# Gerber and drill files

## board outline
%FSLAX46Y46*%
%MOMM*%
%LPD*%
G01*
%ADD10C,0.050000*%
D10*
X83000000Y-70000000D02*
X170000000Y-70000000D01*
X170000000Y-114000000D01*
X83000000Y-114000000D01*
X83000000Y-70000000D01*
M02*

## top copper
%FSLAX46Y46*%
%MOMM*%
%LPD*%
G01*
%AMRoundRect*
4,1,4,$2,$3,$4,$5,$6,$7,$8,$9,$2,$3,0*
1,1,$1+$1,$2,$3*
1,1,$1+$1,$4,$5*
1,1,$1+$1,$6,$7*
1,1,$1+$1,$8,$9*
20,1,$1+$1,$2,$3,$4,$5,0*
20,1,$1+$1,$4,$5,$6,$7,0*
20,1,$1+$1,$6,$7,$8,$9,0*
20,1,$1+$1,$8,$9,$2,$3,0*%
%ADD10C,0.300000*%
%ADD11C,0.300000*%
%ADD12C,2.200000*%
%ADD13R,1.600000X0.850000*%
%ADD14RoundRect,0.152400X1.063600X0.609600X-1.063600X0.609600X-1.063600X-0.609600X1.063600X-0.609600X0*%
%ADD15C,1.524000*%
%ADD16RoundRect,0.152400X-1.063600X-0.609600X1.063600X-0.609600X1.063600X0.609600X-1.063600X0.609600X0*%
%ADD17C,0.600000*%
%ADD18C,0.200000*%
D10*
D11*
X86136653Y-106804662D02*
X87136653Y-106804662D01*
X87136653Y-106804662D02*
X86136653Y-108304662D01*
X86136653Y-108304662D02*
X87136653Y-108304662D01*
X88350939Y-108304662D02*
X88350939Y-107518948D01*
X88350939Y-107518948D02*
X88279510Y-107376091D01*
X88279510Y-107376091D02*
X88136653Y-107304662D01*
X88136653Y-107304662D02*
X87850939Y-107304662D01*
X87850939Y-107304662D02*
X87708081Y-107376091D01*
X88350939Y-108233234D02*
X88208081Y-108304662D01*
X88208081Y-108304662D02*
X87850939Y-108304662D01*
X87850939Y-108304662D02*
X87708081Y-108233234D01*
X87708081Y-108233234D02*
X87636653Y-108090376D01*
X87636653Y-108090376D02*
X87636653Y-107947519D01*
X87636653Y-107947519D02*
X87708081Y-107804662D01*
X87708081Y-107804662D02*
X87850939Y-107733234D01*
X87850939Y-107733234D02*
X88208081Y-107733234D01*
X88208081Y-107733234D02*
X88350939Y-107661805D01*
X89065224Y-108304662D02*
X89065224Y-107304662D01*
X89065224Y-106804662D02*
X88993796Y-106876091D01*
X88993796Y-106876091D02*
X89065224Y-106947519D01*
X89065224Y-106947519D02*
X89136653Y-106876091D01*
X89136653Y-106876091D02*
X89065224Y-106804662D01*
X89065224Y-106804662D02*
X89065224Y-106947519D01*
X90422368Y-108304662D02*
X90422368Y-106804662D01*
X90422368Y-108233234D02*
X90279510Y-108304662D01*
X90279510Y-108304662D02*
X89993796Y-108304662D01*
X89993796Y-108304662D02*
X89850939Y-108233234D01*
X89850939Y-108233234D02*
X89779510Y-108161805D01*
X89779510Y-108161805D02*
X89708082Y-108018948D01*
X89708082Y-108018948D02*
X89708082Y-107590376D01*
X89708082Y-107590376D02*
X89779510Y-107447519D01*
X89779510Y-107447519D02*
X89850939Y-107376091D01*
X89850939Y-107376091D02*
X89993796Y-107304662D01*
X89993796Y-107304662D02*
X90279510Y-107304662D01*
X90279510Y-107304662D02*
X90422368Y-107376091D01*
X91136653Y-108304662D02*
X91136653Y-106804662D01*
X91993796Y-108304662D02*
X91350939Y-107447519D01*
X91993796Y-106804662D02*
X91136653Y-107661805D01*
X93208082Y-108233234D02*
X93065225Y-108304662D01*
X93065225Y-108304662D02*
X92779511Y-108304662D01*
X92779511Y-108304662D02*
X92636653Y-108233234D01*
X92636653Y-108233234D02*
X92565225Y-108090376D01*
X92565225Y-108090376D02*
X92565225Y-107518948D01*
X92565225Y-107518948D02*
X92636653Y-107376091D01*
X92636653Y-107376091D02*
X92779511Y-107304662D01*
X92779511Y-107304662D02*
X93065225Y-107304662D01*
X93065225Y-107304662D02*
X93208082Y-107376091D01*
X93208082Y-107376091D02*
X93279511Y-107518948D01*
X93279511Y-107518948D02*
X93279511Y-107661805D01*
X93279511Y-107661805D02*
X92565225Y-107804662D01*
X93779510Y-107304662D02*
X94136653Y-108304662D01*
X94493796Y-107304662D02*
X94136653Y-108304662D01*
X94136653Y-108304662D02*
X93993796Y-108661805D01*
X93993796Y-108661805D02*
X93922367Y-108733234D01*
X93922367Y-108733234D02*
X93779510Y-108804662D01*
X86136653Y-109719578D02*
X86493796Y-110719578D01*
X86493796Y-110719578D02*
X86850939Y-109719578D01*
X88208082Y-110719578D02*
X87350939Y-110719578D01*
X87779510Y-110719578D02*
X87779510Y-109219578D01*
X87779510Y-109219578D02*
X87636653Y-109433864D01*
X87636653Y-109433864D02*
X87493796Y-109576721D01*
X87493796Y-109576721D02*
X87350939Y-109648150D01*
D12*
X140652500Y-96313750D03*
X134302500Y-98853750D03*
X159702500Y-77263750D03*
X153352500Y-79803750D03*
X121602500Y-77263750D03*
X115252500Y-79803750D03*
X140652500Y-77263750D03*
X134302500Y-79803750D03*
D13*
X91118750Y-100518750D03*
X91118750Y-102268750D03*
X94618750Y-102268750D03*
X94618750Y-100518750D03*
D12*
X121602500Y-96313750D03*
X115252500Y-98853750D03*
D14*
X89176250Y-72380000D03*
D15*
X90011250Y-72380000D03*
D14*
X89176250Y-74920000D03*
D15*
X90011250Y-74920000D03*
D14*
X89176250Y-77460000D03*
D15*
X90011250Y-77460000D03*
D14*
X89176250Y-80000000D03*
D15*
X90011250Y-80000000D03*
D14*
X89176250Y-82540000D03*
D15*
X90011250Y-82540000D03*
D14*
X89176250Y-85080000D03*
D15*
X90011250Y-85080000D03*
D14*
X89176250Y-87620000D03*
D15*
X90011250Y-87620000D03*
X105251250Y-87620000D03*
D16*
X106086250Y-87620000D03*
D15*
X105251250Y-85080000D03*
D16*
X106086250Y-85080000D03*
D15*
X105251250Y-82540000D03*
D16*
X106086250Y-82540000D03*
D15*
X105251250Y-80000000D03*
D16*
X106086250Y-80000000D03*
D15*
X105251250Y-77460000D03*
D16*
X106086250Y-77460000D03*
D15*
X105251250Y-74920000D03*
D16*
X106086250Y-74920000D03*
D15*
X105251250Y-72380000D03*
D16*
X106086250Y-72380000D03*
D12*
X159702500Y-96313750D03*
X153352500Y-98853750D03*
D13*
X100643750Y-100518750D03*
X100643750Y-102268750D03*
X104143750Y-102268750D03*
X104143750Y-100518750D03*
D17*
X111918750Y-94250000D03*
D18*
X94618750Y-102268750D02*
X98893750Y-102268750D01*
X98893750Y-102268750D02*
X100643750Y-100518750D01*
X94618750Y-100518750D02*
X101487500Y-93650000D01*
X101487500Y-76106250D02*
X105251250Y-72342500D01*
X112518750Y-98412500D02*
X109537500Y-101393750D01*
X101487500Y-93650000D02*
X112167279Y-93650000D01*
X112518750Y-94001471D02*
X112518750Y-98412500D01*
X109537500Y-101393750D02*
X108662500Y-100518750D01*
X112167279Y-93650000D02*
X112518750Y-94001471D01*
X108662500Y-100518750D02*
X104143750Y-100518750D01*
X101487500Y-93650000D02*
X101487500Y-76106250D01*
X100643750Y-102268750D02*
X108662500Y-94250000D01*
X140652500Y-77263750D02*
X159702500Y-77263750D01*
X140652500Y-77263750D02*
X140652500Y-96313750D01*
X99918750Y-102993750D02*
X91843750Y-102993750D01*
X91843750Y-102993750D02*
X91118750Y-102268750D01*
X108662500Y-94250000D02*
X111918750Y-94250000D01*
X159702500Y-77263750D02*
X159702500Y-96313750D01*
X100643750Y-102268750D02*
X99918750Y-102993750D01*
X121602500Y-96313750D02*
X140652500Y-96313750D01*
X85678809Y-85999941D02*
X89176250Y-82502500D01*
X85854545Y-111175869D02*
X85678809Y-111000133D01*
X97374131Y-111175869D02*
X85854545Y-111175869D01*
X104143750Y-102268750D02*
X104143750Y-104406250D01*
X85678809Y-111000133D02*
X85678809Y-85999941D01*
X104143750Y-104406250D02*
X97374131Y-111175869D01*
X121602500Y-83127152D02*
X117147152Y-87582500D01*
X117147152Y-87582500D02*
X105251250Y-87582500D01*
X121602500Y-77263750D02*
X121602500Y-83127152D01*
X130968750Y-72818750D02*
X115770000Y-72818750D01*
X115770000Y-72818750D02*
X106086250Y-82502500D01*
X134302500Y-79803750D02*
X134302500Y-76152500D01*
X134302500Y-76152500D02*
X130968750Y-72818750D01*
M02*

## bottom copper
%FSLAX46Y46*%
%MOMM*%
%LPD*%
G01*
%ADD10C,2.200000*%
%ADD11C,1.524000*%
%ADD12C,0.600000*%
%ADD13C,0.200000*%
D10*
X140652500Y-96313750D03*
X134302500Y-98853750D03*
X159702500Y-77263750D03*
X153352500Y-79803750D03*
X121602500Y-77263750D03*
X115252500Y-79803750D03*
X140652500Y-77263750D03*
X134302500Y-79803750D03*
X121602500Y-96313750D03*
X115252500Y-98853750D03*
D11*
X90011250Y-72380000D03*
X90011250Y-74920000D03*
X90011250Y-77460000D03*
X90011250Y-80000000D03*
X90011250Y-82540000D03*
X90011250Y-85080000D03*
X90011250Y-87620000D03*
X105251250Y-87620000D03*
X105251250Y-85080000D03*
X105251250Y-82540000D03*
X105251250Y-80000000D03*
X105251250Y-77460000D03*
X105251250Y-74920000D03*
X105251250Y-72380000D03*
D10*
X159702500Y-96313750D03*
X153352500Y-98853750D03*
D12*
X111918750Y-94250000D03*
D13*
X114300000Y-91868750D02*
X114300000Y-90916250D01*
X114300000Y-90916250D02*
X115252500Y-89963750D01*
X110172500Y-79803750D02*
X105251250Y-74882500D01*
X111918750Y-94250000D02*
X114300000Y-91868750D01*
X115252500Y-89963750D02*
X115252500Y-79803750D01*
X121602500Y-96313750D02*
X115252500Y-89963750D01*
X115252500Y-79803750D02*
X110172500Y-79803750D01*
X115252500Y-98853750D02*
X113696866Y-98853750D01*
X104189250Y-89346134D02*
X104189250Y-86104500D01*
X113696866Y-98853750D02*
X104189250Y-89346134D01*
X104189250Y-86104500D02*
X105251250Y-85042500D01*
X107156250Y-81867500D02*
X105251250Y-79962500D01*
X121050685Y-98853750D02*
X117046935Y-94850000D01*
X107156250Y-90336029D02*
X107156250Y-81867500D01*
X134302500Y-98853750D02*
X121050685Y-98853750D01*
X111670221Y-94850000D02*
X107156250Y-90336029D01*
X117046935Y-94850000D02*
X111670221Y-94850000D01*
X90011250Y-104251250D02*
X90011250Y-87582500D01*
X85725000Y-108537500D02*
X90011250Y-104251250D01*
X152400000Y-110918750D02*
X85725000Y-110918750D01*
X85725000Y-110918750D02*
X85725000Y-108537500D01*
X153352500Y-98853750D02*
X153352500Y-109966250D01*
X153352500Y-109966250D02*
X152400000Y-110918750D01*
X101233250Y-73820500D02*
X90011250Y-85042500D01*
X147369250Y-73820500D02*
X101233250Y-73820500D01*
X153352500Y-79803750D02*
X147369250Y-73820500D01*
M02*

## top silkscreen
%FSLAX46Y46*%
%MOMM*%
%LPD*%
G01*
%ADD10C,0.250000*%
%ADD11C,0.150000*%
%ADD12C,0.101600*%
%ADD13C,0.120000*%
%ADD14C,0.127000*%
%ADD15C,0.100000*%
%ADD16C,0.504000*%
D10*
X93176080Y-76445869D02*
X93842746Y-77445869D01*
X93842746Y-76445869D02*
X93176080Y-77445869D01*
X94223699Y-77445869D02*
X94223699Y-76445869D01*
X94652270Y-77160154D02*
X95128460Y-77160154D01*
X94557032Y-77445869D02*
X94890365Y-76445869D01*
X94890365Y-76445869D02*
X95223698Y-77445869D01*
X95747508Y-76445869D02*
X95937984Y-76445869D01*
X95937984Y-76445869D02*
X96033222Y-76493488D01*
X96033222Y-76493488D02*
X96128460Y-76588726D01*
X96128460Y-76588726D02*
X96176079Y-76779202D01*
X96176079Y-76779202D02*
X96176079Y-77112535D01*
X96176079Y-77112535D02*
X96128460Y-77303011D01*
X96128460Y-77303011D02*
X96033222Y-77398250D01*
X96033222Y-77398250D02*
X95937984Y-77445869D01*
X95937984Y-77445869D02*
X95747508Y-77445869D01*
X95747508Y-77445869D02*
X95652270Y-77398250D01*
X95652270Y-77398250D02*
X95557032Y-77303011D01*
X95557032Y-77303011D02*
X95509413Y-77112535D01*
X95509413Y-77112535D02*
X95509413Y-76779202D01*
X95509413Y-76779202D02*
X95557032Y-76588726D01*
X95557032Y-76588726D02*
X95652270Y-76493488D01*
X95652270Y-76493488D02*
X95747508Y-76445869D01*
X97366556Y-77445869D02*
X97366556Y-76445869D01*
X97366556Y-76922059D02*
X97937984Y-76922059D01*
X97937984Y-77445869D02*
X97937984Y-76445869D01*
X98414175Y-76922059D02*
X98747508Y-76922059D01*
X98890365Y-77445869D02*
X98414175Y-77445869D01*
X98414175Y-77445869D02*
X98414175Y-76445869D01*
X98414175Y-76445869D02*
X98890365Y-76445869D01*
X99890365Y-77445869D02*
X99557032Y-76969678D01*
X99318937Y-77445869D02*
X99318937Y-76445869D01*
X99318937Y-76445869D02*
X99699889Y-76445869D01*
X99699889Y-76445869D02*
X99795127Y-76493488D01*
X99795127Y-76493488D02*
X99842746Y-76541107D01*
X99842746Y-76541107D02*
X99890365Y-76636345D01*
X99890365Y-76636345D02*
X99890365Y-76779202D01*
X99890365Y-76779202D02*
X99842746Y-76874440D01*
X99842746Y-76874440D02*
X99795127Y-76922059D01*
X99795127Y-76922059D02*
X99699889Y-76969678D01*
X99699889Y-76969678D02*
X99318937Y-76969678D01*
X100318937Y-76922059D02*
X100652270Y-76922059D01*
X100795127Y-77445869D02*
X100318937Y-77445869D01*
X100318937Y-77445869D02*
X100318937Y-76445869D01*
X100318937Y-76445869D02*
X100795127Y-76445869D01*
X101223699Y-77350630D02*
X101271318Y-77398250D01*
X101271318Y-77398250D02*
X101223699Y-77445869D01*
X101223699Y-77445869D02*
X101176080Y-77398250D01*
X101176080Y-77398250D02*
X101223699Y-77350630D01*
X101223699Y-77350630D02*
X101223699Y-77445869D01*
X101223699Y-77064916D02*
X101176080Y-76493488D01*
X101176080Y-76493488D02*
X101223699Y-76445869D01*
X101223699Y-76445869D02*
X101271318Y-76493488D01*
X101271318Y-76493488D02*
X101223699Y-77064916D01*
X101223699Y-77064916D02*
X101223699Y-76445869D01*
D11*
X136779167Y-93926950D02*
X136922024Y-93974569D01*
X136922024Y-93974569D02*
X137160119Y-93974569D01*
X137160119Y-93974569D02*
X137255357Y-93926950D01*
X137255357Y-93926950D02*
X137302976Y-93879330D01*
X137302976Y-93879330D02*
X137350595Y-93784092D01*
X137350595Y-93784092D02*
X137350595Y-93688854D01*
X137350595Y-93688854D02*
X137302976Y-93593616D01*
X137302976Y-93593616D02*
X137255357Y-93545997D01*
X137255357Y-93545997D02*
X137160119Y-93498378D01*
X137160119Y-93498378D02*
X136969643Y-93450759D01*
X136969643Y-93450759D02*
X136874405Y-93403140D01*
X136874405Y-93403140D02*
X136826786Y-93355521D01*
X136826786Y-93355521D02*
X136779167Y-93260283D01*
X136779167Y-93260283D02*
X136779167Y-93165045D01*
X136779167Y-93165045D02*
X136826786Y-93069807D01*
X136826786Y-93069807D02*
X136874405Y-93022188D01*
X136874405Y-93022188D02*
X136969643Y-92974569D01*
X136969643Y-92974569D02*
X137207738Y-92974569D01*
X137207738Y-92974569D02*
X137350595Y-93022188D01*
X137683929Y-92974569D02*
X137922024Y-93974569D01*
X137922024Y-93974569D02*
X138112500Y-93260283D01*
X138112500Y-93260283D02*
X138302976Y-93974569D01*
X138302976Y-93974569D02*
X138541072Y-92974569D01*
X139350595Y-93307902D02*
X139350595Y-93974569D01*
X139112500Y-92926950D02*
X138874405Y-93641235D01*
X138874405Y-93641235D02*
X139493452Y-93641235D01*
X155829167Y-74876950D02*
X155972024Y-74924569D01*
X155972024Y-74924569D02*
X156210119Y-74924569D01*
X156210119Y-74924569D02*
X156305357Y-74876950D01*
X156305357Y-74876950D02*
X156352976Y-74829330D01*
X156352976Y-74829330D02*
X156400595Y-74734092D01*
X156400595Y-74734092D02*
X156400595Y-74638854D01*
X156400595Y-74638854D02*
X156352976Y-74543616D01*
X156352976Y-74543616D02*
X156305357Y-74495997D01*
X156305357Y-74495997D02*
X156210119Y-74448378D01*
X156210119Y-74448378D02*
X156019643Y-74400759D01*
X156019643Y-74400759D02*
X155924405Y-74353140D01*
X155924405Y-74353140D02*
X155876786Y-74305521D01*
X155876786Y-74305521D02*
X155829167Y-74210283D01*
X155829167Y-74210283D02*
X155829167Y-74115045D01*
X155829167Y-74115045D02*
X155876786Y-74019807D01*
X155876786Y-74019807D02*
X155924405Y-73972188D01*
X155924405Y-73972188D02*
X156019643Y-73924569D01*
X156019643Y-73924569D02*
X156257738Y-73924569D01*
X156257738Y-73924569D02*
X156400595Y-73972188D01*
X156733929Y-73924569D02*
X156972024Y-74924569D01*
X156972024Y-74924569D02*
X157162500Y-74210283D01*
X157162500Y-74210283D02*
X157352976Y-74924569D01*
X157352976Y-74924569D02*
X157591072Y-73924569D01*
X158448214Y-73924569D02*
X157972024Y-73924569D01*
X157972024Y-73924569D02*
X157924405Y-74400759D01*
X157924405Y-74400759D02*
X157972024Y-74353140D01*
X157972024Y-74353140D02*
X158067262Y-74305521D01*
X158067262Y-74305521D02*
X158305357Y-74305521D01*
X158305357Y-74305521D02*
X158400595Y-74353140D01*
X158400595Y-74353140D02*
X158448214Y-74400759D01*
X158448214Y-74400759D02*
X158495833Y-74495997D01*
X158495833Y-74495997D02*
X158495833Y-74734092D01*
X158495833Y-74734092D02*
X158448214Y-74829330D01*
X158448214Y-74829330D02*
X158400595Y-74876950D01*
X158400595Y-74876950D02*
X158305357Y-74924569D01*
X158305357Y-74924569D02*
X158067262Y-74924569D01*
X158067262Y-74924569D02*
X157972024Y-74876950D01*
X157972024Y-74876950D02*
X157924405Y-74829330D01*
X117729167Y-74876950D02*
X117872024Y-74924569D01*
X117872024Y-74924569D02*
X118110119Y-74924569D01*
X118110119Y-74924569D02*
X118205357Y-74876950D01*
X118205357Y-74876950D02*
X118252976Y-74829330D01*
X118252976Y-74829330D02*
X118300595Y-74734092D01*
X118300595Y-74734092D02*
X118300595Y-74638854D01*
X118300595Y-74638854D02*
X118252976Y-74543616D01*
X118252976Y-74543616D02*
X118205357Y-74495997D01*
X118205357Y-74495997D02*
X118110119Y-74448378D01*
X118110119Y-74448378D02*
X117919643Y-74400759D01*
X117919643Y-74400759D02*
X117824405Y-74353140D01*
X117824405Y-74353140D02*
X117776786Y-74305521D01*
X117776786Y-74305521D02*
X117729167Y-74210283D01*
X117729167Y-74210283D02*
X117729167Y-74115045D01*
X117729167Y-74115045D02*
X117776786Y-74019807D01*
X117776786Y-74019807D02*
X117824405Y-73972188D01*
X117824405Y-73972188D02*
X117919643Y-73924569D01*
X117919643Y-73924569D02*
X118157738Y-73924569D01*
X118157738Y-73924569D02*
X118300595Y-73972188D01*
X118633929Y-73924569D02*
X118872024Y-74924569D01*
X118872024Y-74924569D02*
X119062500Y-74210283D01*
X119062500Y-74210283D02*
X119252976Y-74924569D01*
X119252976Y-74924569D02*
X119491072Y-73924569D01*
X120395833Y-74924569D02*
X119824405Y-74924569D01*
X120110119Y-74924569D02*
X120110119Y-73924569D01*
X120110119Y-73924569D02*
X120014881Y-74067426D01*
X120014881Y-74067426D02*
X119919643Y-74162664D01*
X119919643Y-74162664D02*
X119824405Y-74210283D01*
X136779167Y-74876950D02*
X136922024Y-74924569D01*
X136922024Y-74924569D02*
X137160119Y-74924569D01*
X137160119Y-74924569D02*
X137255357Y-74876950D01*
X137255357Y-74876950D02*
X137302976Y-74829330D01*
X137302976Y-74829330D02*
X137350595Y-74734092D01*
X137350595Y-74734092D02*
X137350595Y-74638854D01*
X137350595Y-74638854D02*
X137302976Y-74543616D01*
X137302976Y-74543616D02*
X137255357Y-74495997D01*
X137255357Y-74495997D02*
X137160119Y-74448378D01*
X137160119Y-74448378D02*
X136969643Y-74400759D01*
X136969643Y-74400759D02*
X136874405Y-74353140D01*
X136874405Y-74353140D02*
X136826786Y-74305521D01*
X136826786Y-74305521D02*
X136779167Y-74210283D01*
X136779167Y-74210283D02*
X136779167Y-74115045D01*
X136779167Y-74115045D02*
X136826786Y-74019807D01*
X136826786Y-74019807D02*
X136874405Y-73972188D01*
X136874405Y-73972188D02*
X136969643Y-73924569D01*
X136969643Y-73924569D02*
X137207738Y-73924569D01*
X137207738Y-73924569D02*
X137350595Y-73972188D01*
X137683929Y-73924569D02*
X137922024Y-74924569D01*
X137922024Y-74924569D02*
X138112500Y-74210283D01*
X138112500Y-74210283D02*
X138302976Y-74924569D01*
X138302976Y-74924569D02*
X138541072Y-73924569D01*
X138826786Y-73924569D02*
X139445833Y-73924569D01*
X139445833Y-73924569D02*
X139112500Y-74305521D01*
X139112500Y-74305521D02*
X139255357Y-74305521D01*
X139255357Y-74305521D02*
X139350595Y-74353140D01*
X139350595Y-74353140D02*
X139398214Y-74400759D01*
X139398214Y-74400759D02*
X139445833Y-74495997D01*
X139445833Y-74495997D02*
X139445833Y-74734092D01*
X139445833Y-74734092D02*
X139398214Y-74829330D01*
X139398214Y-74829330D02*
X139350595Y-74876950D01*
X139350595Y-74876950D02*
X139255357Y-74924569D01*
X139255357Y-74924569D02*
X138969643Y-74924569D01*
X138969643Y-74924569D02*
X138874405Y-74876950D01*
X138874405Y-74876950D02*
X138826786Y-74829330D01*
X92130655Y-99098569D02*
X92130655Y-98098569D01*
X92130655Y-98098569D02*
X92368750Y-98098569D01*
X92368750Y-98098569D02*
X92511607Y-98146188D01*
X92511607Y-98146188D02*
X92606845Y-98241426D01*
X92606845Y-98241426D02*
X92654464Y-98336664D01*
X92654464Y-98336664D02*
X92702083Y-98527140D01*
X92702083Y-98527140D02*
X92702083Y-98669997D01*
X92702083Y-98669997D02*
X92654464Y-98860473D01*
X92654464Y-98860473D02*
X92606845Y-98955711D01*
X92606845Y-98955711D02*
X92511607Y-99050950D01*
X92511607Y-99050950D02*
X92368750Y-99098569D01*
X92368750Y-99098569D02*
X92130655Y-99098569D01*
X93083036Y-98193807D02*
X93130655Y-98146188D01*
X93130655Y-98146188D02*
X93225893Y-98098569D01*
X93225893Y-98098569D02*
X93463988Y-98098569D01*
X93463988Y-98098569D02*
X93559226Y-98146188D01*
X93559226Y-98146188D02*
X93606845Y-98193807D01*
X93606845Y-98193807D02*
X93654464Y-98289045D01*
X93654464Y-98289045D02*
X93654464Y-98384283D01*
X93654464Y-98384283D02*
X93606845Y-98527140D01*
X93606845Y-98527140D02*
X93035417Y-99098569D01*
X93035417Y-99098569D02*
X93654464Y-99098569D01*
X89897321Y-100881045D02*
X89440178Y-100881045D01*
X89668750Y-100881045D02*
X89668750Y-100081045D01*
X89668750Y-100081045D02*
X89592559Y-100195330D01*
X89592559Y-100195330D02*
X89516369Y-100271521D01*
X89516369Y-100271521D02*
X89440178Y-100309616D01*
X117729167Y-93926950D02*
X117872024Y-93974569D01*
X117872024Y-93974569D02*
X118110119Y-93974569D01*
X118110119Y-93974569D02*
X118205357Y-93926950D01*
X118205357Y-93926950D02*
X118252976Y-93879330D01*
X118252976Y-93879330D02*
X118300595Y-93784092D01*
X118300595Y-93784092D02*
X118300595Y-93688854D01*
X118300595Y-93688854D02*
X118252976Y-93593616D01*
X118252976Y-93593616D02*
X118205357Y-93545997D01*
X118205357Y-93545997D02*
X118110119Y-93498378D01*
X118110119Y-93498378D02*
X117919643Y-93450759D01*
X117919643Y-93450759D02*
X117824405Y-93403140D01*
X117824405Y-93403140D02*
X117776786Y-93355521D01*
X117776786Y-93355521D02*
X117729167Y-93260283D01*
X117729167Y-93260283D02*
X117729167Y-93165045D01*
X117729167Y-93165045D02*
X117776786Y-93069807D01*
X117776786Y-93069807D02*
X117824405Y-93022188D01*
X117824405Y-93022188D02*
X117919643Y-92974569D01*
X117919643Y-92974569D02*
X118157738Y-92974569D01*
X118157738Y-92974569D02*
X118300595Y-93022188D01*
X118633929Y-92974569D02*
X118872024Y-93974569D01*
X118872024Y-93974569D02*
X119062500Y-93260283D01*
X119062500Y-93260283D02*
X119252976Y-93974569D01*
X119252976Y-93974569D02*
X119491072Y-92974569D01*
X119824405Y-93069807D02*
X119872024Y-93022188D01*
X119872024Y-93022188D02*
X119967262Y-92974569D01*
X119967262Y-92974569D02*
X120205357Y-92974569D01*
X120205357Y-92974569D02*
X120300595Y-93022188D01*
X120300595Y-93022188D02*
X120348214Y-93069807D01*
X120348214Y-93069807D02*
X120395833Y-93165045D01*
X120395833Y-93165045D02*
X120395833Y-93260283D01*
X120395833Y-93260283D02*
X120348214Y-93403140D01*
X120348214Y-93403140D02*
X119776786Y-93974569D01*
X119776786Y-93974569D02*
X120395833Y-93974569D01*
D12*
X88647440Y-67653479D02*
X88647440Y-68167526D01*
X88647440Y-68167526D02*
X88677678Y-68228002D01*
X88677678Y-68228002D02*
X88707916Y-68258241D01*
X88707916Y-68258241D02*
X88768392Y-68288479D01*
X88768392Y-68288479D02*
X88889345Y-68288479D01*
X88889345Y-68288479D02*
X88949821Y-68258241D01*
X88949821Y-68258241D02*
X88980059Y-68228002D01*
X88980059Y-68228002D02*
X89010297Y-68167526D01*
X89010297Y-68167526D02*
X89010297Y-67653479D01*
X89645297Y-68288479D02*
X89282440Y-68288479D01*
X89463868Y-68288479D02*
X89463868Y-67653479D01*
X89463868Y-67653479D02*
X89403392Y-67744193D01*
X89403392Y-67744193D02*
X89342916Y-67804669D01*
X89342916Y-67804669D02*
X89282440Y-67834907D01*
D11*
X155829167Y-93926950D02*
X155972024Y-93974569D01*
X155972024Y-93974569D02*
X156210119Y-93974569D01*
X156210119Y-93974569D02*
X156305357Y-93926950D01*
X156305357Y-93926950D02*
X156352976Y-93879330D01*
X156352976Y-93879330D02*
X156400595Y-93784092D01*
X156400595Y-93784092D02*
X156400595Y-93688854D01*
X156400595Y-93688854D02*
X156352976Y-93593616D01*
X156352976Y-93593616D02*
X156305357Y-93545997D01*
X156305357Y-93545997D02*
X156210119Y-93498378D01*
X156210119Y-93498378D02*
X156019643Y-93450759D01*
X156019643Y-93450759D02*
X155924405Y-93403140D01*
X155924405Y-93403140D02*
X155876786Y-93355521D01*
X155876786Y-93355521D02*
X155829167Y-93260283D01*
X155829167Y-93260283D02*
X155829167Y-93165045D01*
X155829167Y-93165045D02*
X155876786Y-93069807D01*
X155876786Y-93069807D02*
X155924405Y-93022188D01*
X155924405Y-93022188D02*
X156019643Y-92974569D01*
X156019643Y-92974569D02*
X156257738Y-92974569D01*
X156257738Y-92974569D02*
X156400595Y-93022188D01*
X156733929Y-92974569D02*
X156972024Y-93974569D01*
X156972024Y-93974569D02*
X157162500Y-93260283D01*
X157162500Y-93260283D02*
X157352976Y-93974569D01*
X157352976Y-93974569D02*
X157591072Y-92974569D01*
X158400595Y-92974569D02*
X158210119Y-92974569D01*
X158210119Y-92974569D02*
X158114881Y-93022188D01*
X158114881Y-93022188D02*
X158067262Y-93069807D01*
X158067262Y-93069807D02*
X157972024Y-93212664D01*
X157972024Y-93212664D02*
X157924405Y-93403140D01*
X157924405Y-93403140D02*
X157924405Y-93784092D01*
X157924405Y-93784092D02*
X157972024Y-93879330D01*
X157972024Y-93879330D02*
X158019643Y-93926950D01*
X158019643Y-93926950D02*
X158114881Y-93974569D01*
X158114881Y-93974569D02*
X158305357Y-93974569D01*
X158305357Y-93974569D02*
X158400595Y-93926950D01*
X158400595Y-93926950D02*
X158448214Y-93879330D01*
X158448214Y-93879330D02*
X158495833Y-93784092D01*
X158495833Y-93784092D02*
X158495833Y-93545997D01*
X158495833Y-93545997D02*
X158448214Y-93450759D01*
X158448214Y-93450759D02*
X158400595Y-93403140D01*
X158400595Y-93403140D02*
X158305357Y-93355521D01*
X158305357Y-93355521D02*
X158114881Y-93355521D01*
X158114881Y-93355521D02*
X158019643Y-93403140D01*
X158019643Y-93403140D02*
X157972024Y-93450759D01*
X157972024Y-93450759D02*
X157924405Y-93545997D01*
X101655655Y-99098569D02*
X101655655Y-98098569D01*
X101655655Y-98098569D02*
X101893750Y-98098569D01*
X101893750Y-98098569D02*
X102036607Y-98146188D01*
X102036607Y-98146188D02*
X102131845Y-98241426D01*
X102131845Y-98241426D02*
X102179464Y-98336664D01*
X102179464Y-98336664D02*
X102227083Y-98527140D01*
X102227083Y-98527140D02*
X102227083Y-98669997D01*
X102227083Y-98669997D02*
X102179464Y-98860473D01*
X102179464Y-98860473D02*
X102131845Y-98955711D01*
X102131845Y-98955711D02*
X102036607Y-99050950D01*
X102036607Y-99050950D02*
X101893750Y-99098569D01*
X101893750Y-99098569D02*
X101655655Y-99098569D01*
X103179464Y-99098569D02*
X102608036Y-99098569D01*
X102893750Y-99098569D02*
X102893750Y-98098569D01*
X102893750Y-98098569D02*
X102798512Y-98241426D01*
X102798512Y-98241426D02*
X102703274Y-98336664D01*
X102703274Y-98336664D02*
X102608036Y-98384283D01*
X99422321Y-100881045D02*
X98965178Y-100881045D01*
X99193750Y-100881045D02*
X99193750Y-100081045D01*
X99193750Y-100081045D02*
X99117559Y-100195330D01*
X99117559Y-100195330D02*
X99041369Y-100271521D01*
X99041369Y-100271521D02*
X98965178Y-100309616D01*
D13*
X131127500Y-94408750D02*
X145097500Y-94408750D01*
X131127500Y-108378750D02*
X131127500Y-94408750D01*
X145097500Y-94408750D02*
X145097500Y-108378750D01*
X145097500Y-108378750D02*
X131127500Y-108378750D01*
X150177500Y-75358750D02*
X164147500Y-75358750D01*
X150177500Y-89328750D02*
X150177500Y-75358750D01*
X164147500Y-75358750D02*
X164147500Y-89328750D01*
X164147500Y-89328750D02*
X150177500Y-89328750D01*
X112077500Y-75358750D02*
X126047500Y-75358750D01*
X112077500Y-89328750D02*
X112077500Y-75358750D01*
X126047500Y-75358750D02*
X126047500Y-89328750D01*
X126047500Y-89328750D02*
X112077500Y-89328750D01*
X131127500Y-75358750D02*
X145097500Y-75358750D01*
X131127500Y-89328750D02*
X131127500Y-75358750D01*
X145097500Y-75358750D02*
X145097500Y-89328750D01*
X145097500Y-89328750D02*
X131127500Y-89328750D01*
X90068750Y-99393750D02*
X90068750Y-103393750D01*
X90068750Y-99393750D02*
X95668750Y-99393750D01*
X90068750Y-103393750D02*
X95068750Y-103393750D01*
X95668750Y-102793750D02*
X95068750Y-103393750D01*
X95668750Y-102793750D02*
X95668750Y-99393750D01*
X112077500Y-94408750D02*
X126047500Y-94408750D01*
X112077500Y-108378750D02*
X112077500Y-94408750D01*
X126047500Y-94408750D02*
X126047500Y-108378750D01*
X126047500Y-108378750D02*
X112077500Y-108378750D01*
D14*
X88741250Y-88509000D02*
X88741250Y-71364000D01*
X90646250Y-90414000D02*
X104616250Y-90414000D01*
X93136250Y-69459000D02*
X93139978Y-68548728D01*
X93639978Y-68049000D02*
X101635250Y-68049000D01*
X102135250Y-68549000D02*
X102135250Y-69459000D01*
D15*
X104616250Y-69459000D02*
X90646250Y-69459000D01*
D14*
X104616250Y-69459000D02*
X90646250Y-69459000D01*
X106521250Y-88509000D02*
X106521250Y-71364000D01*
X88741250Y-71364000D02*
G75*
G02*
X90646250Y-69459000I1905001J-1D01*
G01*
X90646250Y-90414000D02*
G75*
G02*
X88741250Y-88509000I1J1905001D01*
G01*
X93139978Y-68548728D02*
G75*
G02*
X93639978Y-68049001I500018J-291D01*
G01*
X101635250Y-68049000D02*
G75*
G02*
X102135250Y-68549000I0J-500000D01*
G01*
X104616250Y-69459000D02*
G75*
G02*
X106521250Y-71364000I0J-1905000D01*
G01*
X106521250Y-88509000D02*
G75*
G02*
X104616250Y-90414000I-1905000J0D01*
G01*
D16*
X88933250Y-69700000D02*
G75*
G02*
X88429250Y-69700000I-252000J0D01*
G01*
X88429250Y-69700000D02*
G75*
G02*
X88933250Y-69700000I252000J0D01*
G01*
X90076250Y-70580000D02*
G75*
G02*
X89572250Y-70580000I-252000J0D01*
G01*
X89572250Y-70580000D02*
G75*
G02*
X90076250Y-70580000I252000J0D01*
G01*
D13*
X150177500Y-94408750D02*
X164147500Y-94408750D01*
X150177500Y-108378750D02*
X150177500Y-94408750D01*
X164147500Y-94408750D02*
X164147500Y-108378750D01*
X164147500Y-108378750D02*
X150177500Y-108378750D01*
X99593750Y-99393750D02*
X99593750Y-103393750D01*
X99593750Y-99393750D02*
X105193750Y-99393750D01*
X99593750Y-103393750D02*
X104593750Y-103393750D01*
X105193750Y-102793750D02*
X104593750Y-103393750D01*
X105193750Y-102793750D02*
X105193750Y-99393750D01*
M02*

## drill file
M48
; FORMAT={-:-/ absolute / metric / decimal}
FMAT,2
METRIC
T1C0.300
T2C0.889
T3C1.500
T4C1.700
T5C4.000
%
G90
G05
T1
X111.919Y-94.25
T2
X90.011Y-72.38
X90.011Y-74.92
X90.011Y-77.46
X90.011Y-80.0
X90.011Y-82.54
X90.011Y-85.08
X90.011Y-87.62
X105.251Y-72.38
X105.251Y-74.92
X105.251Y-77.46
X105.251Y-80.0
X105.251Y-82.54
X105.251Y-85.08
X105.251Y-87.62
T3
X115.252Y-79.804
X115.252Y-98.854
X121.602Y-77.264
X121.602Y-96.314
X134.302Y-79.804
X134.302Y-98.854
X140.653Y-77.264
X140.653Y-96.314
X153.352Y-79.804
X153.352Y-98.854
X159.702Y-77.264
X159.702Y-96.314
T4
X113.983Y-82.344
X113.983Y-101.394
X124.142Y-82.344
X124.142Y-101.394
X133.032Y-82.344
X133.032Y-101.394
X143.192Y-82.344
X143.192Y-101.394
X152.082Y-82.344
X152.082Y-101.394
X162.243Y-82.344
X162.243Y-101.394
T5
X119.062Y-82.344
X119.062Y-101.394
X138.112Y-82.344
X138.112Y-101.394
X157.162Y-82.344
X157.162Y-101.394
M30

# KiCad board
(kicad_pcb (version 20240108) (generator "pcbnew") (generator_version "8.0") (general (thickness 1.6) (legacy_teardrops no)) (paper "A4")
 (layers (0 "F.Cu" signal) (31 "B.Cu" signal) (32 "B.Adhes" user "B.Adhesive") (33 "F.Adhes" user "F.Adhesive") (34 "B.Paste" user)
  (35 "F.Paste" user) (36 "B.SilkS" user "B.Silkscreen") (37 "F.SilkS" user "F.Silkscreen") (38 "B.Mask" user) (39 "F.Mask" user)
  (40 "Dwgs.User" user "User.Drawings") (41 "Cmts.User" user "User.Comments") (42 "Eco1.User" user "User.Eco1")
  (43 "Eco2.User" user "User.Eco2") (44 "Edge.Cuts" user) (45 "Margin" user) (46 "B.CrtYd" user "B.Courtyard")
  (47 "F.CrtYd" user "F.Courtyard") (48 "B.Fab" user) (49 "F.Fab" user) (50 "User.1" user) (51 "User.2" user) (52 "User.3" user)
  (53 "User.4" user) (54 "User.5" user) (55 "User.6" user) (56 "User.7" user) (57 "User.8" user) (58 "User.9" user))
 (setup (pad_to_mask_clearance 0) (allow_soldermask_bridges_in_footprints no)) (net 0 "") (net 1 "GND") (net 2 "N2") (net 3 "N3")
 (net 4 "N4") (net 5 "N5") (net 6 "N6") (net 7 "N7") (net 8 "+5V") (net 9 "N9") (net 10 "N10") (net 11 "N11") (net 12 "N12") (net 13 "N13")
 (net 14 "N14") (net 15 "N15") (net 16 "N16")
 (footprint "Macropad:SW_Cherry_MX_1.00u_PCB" (layer "F.Cu") (at 140.6525 96.31375)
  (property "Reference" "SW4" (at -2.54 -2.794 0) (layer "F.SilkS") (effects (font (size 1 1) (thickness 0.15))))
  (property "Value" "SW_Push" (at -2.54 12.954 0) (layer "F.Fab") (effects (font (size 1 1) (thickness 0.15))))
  (fp_line (start -9.525 -1.905) (end 4.445 -1.905) (stroke (width 0.12) (type solid)) (layer "F.SilkS"))
  (fp_line (start -9.525 12.065) (end -9.525 -1.905) (stroke (width 0.12) (type solid)) (layer "F.SilkS"))
  (fp_line (start 4.445 -1.905) (end 4.445 12.065) (stroke (width 0.12) (type solid)) (layer "F.SilkS"))
  (fp_line (start 4.445 12.065) (end -9.525 12.065) (stroke (width 0.12) (type solid)) (layer "F.SilkS"))
  (pad "" np_thru_hole circle (at -7.62 5.08) (size 1.7 1.7) (drill 1.7) (layers "*.Cu" "*.Mask"))
  (pad "" np_thru_hole circle (at -2.54 5.08) (size 4 4) (drill 4) (layers "*.Cu" "*.Mask"))
  (pad "" np_thru_hole circle (at 2.54 5.08) (size 1.7 1.7) (drill 1.7) (layers "*.Cu" "*.Mask"))
  (pad "1" thru_hole circle (at 0 0) (size 2.2 2.2) (drill 1.5) (layers "*.Cu" "*.Mask") (remove_unused_layers no) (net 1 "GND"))
  (pad "2" thru_hole circle (at -6.35 2.54) (size 2.2 2.2) (drill 1.5) (layers "*.Cu" "*.Mask") (remove_unused_layers no) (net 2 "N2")))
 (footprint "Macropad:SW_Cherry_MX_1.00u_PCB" (layer "F.Cu") (at 159.7025 77.26375)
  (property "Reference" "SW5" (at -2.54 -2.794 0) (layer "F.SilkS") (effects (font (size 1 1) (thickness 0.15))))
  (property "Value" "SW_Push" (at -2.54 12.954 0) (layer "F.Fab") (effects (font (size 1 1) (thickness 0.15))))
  (fp_line (start -9.525 -1.905) (end 4.445 -1.905) (stroke (width 0.12) (type solid)) (layer "F.SilkS"))
  (fp_line (start -9.525 12.065) (end -9.525 -1.905) (stroke (width 0.12) (type solid)) (layer "F.SilkS"))
  (fp_line (start 4.445 -1.905) (end 4.445 12.065) (stroke (width 0.12) (type solid)) (layer "F.SilkS"))
  (fp_line (start 4.445 12.065) (end -9.525 12.065) (stroke (width 0.12) (type solid)) (layer "F.SilkS"))
  (pad "" np_thru_hole circle (at -7.62 5.08) (size 1.7 1.7) (drill 1.7) (layers "*.Cu" "*.Mask"))
  (pad "" np_thru_hole circle (at -2.54 5.08) (size 4 4) (drill 4) (layers "*.Cu" "*.Mask"))
  (pad "" np_thru_hole circle (at 2.54 5.08) (size 1.7 1.7) (drill 1.7) (layers "*.Cu" "*.Mask"))
  (pad "1" thru_hole circle (at 0 0) (size 2.2 2.2) (drill 1.5) (layers "*.Cu" "*.Mask") (remove_unused_layers no) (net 1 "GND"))
  (pad "2" thru_hole circle (at -6.35 2.54) (size 2.2 2.2) (drill 1.5) (layers "*.Cu" "*.Mask") (remove_unused_layers no) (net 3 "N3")))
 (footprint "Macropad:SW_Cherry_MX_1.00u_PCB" (layer "F.Cu") (at 121.6025 77.26375)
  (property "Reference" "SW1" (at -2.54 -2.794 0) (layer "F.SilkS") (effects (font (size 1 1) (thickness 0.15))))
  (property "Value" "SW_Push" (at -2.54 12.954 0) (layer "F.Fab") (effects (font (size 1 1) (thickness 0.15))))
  (fp_line (start -9.525 -1.905) (end 4.445 -1.905) (stroke (width 0.12) (type solid)) (layer "F.SilkS"))
  (fp_line (start -9.525 12.065) (end -9.525 -1.905) (stroke (width 0.12) (type solid)) (layer "F.SilkS"))
  (fp_line (start 4.445 -1.905) (end 4.445 12.065) (stroke (width 0.12) (type solid)) (layer "F.SilkS"))
  (fp_line (start 4.445 12.065) (end -9.525 12.065) (stroke (width 0.12) (type solid)) (layer "F.SilkS"))
  (pad "" np_thru_hole circle (at -7.62 5.08) (size 1.7 1.7) (drill 1.7) (layers "*.Cu" "*.Mask"))
  (pad "" np_thru_hole circle (at -2.54 5.08) (size 4 4) (drill 4) (layers "*.Cu" "*.Mask"))
  (pad "" np_thru_hole circle (at 2.54 5.08) (size 1.7 1.7) (drill 1.7) (layers "*.Cu" "*.Mask"))
  (pad "1" thru_hole circle (at 0 0) (size 2.2 2.2) (drill 1.5) (layers "*.Cu" "*.Mask") (remove_unused_layers no) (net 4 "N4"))
  (pad "2" thru_hole circle (at -6.35 2.54) (size 2.2 2.2) (drill 1.5) (layers "*.Cu" "*.Mask") (remove_unused_layers no) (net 1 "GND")))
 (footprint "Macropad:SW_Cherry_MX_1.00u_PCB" (layer "F.Cu") (at 140.6525 77.26375)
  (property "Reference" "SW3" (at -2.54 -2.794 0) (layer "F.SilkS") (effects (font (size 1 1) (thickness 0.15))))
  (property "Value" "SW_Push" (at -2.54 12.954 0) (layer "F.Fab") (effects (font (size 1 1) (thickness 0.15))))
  (fp_line (start -9.525 -1.905) (end 4.445 -1.905) (stroke (width 0.12) (type solid)) (layer "F.SilkS"))
  (fp_line (start -9.525 12.065) (end -9.525 -1.905) (stroke (width 0.12) (type solid)) (layer "F.SilkS"))
  (fp_line (start 4.445 -1.905) (end 4.445 12.065) (stroke (width 0.12) (type solid)) (layer "F.SilkS"))
  (fp_line (start 4.445 12.065) (end -9.525 12.065) (stroke (width 0.12) (type solid)) (layer "F.SilkS"))
  (pad "" np_thru_hole circle (at -7.62 5.08) (size 1.7 1.7) (drill 1.7) (layers "*.Cu" "*.Mask"))
  (pad "" np_thru_hole circle (at -2.54 5.08) (size 4 4) (drill 4) (layers "*.Cu" "*.Mask"))
  (pad "" np_thru_hole circle (at 2.54 5.08) (size 1.7 1.7) (drill 1.7) (layers "*.Cu" "*.Mask"))
  (pad "1" thru_hole circle (at 0 0) (size 2.2 2.2) (drill 1.5) (layers "*.Cu" "*.Mask") (remove_unused_layers no) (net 1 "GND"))
  (pad "2" thru_hole circle (at -6.35 2.54) (size 2.2 2.2) (drill 1.5) (layers "*.Cu" "*.Mask") (remove_unused_layers no) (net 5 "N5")))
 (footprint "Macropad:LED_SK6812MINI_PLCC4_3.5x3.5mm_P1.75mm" (layer "F.Cu") (at 92.86875 101.39375)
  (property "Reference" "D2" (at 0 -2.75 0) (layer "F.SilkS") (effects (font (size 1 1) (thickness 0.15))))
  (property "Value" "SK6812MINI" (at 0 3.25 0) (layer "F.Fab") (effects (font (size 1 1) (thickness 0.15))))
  (fp_line (start -2.8 -2) (end -2.8 2) (stroke (width 0.12) (type default)) (layer "F.SilkS"))
  (fp_line (start -2.8 -2) (end 2.8 -2) (stroke (width 0.12) (type solid)) (layer "F.SilkS"))
  (fp_line (start -2.8 2) (end 2.2 2) (stroke (width 0.12) (type solid)) (layer "F.SilkS"))
  (fp_line (start 2.8 1.4) (end 2.2 2) (stroke (width 0.12) (type default)) (layer "F.SilkS"))
  (fp_line (start 2.8 1.4) (end 2.8 -2) (stroke (width 0.12) (type solid)) (layer "F.SilkS"))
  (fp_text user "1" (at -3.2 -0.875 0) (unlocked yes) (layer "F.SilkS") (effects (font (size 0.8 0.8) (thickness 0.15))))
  (pad "1" smd rect (at -1.75 -0.875) (size 1.6 0.85) (layers "F.Cu" "F.Paste" "F.Mask") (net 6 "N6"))
  (pad "2" smd rect (at -1.75 0.875) (size 1.6 0.85) (layers "F.Cu" "F.Paste" "F.Mask") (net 1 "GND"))
  (pad "3" smd rect (at 1.75 0.875) (size 1.6 0.85) (layers "F.Cu" "F.Paste" "F.Mask") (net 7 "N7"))
  (pad "4" smd rect (at 1.75 -0.875) (size 1.6 0.85) (layers "F.Cu" "F.Paste" "F.Mask") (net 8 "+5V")))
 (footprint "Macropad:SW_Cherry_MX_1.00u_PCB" (layer "F.Cu") (at 121.6025 96.31375)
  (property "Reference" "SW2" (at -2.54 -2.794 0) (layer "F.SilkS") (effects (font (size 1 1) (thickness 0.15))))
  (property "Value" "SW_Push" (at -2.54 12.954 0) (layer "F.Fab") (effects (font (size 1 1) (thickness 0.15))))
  (fp_line (start -9.525 -1.905) (end 4.445 -1.905) (stroke (width 0.12) (type solid)) (layer "F.SilkS"))
  (fp_line (start -9.525 12.065) (end -9.525 -1.905) (stroke (width 0.12) (type solid)) (layer "F.SilkS"))
  (fp_line (start 4.445 -1.905) (end 4.445 12.065) (stroke (width 0.12) (type solid)) (layer "F.SilkS"))
  (fp_line (start 4.445 12.065) (end -9.525 12.065) (stroke (width 0.12) (type solid)) (layer "F.SilkS"))
  (pad "" np_thru_hole circle (at -7.62 5.08) (size 1.7 1.7) (drill 1.7) (layers "*.Cu" "*.Mask"))
  (pad "" np_thru_hole circle (at -2.54 5.08) (size 4 4) (drill 4) (layers "*.Cu" "*.Mask"))
  (pad "" np_thru_hole circle (at 2.54 5.08) (size 1.7 1.7) (drill 1.7) (layers "*.Cu" "*.Mask"))
  (pad "1" thru_hole circle (at 0 0) (size 2.2 2.2) (drill 1.5) (layers "*.Cu" "*.Mask") (remove_unused_layers no) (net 1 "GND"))
  (pad "2" thru_hole circle (at -6.35 2.54) (size 2.2 2.2) (drill 1.5) (layers "*.Cu" "*.Mask") (remove_unused_layers no) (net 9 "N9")))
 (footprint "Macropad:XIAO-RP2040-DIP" (layer "F.Cu") (at 97.63125 80)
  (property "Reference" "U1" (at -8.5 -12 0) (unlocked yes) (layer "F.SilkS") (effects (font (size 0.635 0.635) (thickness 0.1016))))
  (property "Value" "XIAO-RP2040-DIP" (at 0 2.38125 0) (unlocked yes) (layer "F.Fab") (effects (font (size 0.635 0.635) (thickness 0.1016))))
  (fp_line (start -8.89 8.509) (end -8.89 -8.636) (stroke (width 0.127) (type solid)) (layer "F.SilkS"))
  (fp_line (start -6.985 10.414) (end 6.985 10.414) (stroke (width 0.127) (type solid)) (layer "F.SilkS"))
  (fp_line (start -4.495 -10.541) (end -4.491272 -11.451272) (stroke (width 0.127) (type solid)) (layer "F.SilkS"))
  (fp_line (start -3.991272 -11.951) (end 4.004 -11.951) (stroke (width 0.127) (type solid)) (layer "F.SilkS"))
  (fp_line (start 4.504 -11.451) (end 4.504 -10.541) (stroke (width 0.127) (type solid)) (layer "F.SilkS"))
  (fp_line (start 6.985 -10.541) (end -6.985 -10.541) (stroke (width 0.1) (type solid)) (layer "F.SilkS"))
  (fp_line (start 6.985 -10.541) (end -6.985 -10.541) (stroke (width 0.127) (type solid)) (layer "F.SilkS"))
  (fp_line (start 8.89 8.509) (end 8.89 -8.636) (stroke (width 0.127) (type solid)) (layer "F.SilkS"))
  (fp_arc (start -8.89 -8.636) (mid -8.332038 -9.983038) (end -6.985 -10.541) (stroke (width 0.127) (type solid)) (layer "F.SilkS"))
  (fp_arc (start -6.985 10.414) (mid -8.332038 9.856038) (end -8.89 8.509) (stroke (width 0.127) (type solid)) (layer "F.SilkS"))
  (fp_arc (start -4.491272 -11.451272) (mid -4.344724 -11.804644) (end -3.991272 -11.951) (stroke (width 0.127) (type default))
   (layer "F.SilkS"))
  (fp_arc (start 4.004 -11.951) (mid 4.357553 -11.804553) (end 4.504 -11.451) (stroke (width 0.127) (type default)) (layer "F.SilkS"))
  (fp_arc (start 6.985 -10.541) (mid 8.332038 -9.983038) (end 8.89 -8.636) (stroke (width 0.127) (type solid)) (layer "F.SilkS"))
  (fp_arc (start 8.89 8.509) (mid 8.332038 9.856038) (end 6.985 10.414) (stroke (width 0.127) (type solid)) (layer "F.SilkS"))
  (fp_circle (center -8.95 -10.3) (end -8.95 -10.554) (stroke (width 0.5) (type solid)) (fill solid) (layer "F.SilkS"))
  (fp_circle (center -7.807 -9.42) (end -7.807 -9.674) (stroke (width 0.5) (type solid)) (fill solid) (layer "F.SilkS"))
  (pad "1" smd roundrect (at -8.455 -7.62 180) (size 2.432 1.524) (layers "F.Cu" "F.Mask") (roundrect_rratio 0.1) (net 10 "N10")
   (thermal_bridge_angle 45))
  (pad "1" thru_hole circle (at -7.62 -7.62 180) (size 1.524 1.524) (drill 0.889) (layers "*.Cu" "*.Mask") (remove_unused_layers no)
   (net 10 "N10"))
  (pad "2" smd roundrect (at -8.455 -5.08 180) (size 2.432 1.524) (layers "F.Cu" "F.Mask") (roundrect_rratio 0.1) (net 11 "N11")
   (thermal_bridge_angle 45))
  (pad "2" thru_hole circle (at -7.62 -5.08 180) (size 1.524 1.524) (drill 0.889) (layers "*.Cu" "*.Mask") (remove_unused_layers no)
   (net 11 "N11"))
  (pad "3" smd roundrect (at -8.455 -2.54 180) (size 2.432 1.524) (layers "F.Cu" "F.Mask") (roundrect_rratio 0.1) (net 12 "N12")
   (thermal_bridge_angle 45))
  (pad "3" thru_hole circle (at -7.62 -2.54 180) (size 1.524 1.524) (drill 0.889) (layers "*.Cu" "*.Mask") (remove_unused_layers no)
   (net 12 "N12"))
  (pad "4" smd roundrect (at -8.455 0 180) (size 2.432 1.524) (layers "F.Cu" "F.Mask") (roundrect_rratio 0.1) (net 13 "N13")
   (thermal_bridge_angle 45))
  (pad "4" thru_hole circle (at -7.62 0 180) (size 1.524 1.524) (drill 0.889) (layers "*.Cu" "*.Mask") (remove_unused_layers no)
   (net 13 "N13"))
  (pad "5" smd roundrect (at -8.455 2.54 180) (size 2.432 1.524) (layers "F.Cu" "F.Mask") (roundrect_rratio 0.1) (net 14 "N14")
   (thermal_bridge_angle 45))
  (pad "5" thru_hole circle (at -7.62 2.54 180) (size 1.524 1.524) (drill 0.889) (layers "*.Cu" "*.Mask") (remove_unused_layers no)
   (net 14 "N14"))
  (pad "6" smd roundrect (at -8.455 5.08 180) (size 2.432 1.524) (layers "F.Cu" "F.Mask") (roundrect_rratio 0.1) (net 3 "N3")
   (thermal_bridge_angle 45))
  (pad "6" thru_hole circle (at -7.62 5.08 180) (size 1.524 1.524) (drill 0.889) (layers "*.Cu" "*.Mask") (remove_unused_layers no)
   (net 3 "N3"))
  (pad "7" smd roundrect (at -8.455 7.62 180) (size 2.432 1.524) (layers "F.Cu" "F.Mask") (roundrect_rratio 0.1) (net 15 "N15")
   (thermal_bridge_angle 45))
  (pad "7" thru_hole circle (at -7.62 7.62 180) (size 1.524 1.524) (drill 0.889) (layers "*.Cu" "*.Mask") (remove_unused_layers no)
   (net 15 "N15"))
  (pad "8" thru_hole circle (at 7.62 7.62) (size 1.524 1.524) (drill 0.889) (layers "*.Cu" "*.Mask") (remove_unused_layers no) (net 4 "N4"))
  (pad "8" smd roundrect (at 8.455 7.62) (size 2.432 1.524) (layers "F.Cu" "F.Mask") (roundrect_rratio 0.1) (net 4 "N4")
   (thermal_bridge_angle 45))
  (pad "9" thru_hole circle (at 7.62 5.08) (size 1.524 1.524) (drill 0.889) (layers "*.Cu" "*.Mask") (remove_unused_layers no) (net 9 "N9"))
  (pad "9" smd roundrect (at 8.455 5.08) (size 2.432 1.524) (layers "F.Cu" "F.Mask") (roundrect_rratio 0.1) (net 9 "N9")
   (thermal_bridge_angle 45))
  (pad "10" thru_hole circle (at 7.62 2.54) (size 1.524 1.524) (drill 0.889) (layers "*.Cu" "*.Mask") (remove_unused_layers no) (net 5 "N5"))
  (pad "10" smd roundrect (at 8.455 2.54) (size 2.432 1.524) (layers "F.Cu" "F.Mask") (roundrect_rratio 0.1) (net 5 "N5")
   (thermal_bridge_angle 45))
  (pad "11" thru_hole circle (at 7.62 0) (size 1.524 1.524) (drill 0.889) (layers "*.Cu" "*.Mask") (remove_unused_layers no) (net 2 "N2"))
  (pad "11" smd roundrect (at 8.455 0) (size 2.432 1.524) (layers "F.Cu" "F.Mask") (roundrect_rratio 0.1) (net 2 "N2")
   (thermal_bridge_angle 45))
  (pad "12" thru_hole circle (at 7.62 -2.54) (size 1.524 1.524) (drill 0.889) (layers "*.Cu" "*.Mask") (remove_unused_layers no)
   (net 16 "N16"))
  (pad "12" smd roundrect (at 8.455 -2.54) (size 2.432 1.524) (layers "F.Cu" "F.Mask") (roundrect_rratio 0.1) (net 16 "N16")
   (thermal_bridge_angle 45))
  (pad "13" thru_hole circle (at 7.62 -5.08) (size 1.524 1.524) (drill 0.889) (layers "*.Cu" "*.Mask") (remove_unused_layers no)
   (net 1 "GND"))
  (pad "13" smd roundrect (at 8.455 -5.08) (size 2.432 1.524) (layers "F.Cu" "F.Mask") (roundrect_rratio 0.1) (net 1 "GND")
   (thermal_bridge_angle 45))
  (pad "14" thru_hole circle (at 7.62 -7.62) (size 1.524 1.524) (drill 0.889) (layers "*.Cu" "*.Mask") (remove_unused_layers no)
   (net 8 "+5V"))
  (pad "14" smd roundrect (at 8.455 -7.62) (size 2.432 1.524) (layers "F.Cu" "F.Mask") (roundrect_rratio 0.1) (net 8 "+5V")
   (thermal_bridge_angle 45)))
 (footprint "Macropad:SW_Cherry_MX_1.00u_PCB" (layer "F.Cu") (at 159.7025 96.31375)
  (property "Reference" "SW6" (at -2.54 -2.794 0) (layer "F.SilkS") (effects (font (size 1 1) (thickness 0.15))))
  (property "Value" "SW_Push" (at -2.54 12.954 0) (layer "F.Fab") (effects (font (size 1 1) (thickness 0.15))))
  (fp_line (start -9.525 -1.905) (end 4.445 -1.905) (stroke (width 0.12) (type solid)) (layer "F.SilkS"))
  (fp_line (start -9.525 12.065) (end -9.525 -1.905) (stroke (width 0.12) (type solid)) (layer "F.SilkS"))
  (fp_line (start 4.445 -1.905) (end 4.445 12.065) (stroke (width 0.12) (type solid)) (layer "F.SilkS"))
  (fp_line (start 4.445 12.065) (end -9.525 12.065) (stroke (width 0.12) (type solid)) (layer "F.SilkS"))
  (pad "" np_thru_hole circle (at -7.62 5.08) (size 1.7 1.7) (drill 1.7) (layers "*.Cu" "*.Mask"))
  (pad "" np_thru_hole circle (at -2.54 5.08) (size 4 4) (drill 4) (layers "*.Cu" "*.Mask"))
  (pad "" np_thru_hole circle (at 2.54 5.08) (size 1.7 1.7) (drill 1.7) (layers "*.Cu" "*.Mask"))
  (pad "1" thru_hole circle (at 0 0) (size 2.2 2.2) (drill 1.5) (layers "*.Cu" "*.Mask") (remove_unused_layers no) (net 1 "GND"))
  (pad "2" thru_hole circle (at -6.35 2.54) (size 2.2 2.2) (drill 1.5) (layers "*.Cu" "*.Mask") (remove_unused_layers no) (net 15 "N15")))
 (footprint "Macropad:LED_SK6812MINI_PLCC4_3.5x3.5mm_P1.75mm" (layer "F.Cu") (at 102.39375 101.39375)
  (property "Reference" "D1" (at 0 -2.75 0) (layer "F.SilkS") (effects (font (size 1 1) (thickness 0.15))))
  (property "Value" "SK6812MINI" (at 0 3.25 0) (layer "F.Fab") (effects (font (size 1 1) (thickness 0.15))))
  (fp_line (start -2.8 -2) (end -2.8 2) (stroke (width 0.12) (type default)) (layer "F.SilkS"))
  (fp_line (start -2.8 -2) (end 2.8 -2) (stroke (width 0.12) (type solid)) (layer "F.SilkS"))
  (fp_line (start -2.8 2) (end 2.2 2) (stroke (width 0.12) (type solid)) (layer "F.SilkS"))
  (fp_line (start 2.8 1.4) (end 2.2 2) (stroke (width 0.12) (type default)) (layer "F.SilkS"))
  (fp_line (start 2.8 1.4) (end 2.8 -2) (stroke (width 0.12) (type solid)) (layer "F.SilkS"))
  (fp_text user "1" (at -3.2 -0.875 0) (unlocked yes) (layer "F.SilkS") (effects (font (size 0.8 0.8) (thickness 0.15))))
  (pad "1" smd rect (at -1.75 -0.875) (size 1.6 0.85) (layers "F.Cu" "F.Paste" "F.Mask") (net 7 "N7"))
  (pad "2" smd rect (at -1.75 0.875) (size 1.6 0.85) (layers "F.Cu" "F.Paste" "F.Mask") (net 1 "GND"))
  (pad "3" smd rect (at 1.75 0.875) (size 1.6 0.85) (layers "F.Cu" "F.Paste" "F.Mask") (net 14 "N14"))
  (pad "4" smd rect (at 1.75 -0.875) (size 1.6 0.85) (layers "F.Cu" "F.Paste" "F.Mask") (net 8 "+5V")))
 (gr_rect (start 83 70) (end 170 114) (stroke (width 0.05) (type default)) (fill none) (layer "Edge.Cuts"))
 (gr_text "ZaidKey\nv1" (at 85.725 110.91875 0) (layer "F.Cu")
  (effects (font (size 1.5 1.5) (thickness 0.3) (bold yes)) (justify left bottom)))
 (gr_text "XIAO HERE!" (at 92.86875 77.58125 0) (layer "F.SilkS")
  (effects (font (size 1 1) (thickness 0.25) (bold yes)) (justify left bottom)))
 (segment (start 94.61875 102.26875) (end 98.89375 102.26875) (width 0.2) (layer "F.Cu") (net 7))
 (segment (start 98.89375 102.26875) (end 100.64375 100.51875) (width 0.2) (layer "F.Cu") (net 7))
 (segment (start 94.61875 100.51875) (end 101.4875 93.65) (width 0.2) (layer "F.Cu") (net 8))
 (segment (start 101.4875 76.10625) (end 105.25125 72.3425) (width 0.2) (layer "F.Cu") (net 8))
 (segment (start 112.51875 98.4125) (end 109.5375 101.39375) (width 0.2) (layer "F.Cu") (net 8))
 (segment (start 101.4875 93.65) (end 112.167279 93.65) (width 0.2) (layer "F.Cu") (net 8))
 (segment (start 112.51875 94.001471) (end 112.51875 98.4125) (width 0.2) (layer "F.Cu") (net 8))
 (segment (start 109.5375 101.39375) (end 108.6625 100.51875) (width 0.2) (layer "F.Cu") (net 8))
 (segment (start 112.167279 93.65) (end 112.51875 94.001471) (width 0.2) (layer "F.Cu") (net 8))
 (segment (start 108.6625 100.51875) (end 104.14375 100.51875) (width 0.2) (layer "F.Cu") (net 8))
 (segment (start 101.4875 93.65) (end 101.4875 76.10625) (width 0.2) (layer "F.Cu") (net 8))
 (segment (start 100.64375 102.26875) (end 108.6625 94.25) (width 0.2) (layer "F.Cu") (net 1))
 (segment (start 140.6525 77.26375) (end 159.7025 77.26375) (width 0.2) (layer "F.Cu") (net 1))
 (segment (start 140.6525 77.26375) (end 140.6525 96.31375) (width 0.2) (layer "F.Cu") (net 1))
 (segment (start 99.91875 102.99375) (end 91.84375 102.99375) (width 0.2) (layer "F.Cu") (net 1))
 (segment (start 91.84375 102.99375) (end 91.11875 102.26875) (width 0.2) (layer "F.Cu") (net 1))
 (segment (start 108.6625 94.25) (end 111.91875 94.25) (width 0.2) (layer "F.Cu") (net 1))
 (segment (start 159.7025 77.26375) (end 159.7025 96.31375) (width 0.2) (layer "F.Cu") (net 1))
 (segment (start 100.64375 102.26875) (end 99.91875 102.99375) (width 0.2) (layer "F.Cu") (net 1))
 (segment (start 121.6025 96.31375) (end 140.6525 96.31375) (width 0.2) (layer "F.Cu") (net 1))
 (via (at 111.91875 94.25) (size 0.6) (drill 0.3) (layers "F.Cu" "B.Cu") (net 1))
 (segment (start 114.3 91.86875) (end 114.3 90.91625) (width 0.2) (layer "B.Cu") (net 1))
 (segment (start 114.3 90.91625) (end 115.2525 89.96375) (width 0.2) (layer "B.Cu") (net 1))
 (segment (start 110.1725 79.80375) (end 105.25125 74.8825) (width 0.2) (layer "B.Cu") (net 1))
 (segment (start 111.91875 94.25) (end 114.3 91.86875) (width 0.2) (layer "B.Cu") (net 1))
 (segment (start 115.2525 89.96375) (end 115.2525 79.80375) (width 0.2) (layer "B.Cu") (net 1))
 (segment (start 121.6025 96.31375) (end 115.2525 89.96375) (width 0.2) (layer "B.Cu") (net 1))
 (segment (start 115.2525 79.80375) (end 110.1725 79.80375) (width 0.2) (layer "B.Cu") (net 1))
 (segment (start 85.678809 85.999941) (end 89.17625 82.5025) (width 0.2) (layer "F.Cu") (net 14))
 (segment (start 85.854545 111.175869) (end 85.678809 111.000133) (width 0.2) (layer "F.Cu") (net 14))
 (segment (start 97.374131 111.175869) (end 85.854545 111.175869) (width 0.2) (layer "F.Cu") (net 14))
 (segment (start 104.14375 102.26875) (end 104.14375 104.40625) (width 0.2) (layer "F.Cu") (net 14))
 (segment (start 85.678809 111.000133) (end 85.678809 85.999941) (width 0.2) (layer "F.Cu") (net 14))
 (segment (start 104.14375 104.40625) (end 97.374131 111.175869) (width 0.2) (layer "F.Cu") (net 14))
 (segment (start 121.6025 83.127152) (end 117.147152 87.5825) (width 0.2) (layer "F.Cu") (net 4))
 (segment (start 117.147152 87.5825) (end 105.25125 87.5825) (width 0.2) (layer "F.Cu") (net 4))
 (segment (start 121.6025 77.26375) (end 121.6025 83.127152) (width 0.2) (layer "F.Cu") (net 4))
 (segment (start 115.2525 98.85375) (end 113.696866 98.85375) (width 0.2) (layer "B.Cu") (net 9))
 (segment (start 104.18925 89.346134) (end 104.18925 86.1045) (width 0.2) (layer "B.Cu") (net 9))
 (segment (start 113.696866 98.85375) (end 104.18925 89.346134) (width 0.2) (layer "B.Cu") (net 9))
 (segment (start 104.18925 86.1045) (end 105.25125 85.0425) (width 0.2) (layer "B.Cu") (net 9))
 (segment (start 107.15625 81.8675) (end 105.25125 79.9625) (width 0.2) (layer "B.Cu") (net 2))
 (segment (start 121.050685 98.85375) (end 117.046935 94.85) (width 0.2) (layer "B.Cu") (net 2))
 (segment (start 107.15625 90.336029) (end 107.15625 81.8675) (width 0.2) (layer "B.Cu") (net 2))
 (segment (start 134.3025 98.85375) (end 121.050685 98.85375) (width 0.2) (layer "B.Cu") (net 2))
 (segment (start 111.670221 94.85) (end 107.15625 90.336029) (width 0.2) (layer "B.Cu") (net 2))
 (segment (start 117.046935 94.85) (end 111.670221 94.85) (width 0.2) (layer "B.Cu") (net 2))
 (segment (start 90.01125 104.25125) (end 90.01125 87.5825) (width 0.2) (layer "B.Cu") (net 15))
 (segment (start 85.725 108.5375) (end 90.01125 104.25125) (width 0.2) (layer "B.Cu") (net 15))
 (segment (start 152.4 110.91875) (end 85.725 110.91875) (width 0.2) (layer "B.Cu") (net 15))
 (segment (start 85.725 110.91875) (end 85.725 108.5375) (width 0.2) (layer "B.Cu") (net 15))
 (segment (start 153.3525 98.85375) (end 153.3525 109.96625) (width 0.2) (layer "B.Cu") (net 15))
 (segment (start 153.3525 109.96625) (end 152.4 110.91875) (width 0.2) (layer "B.Cu") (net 15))
 (segment (start 130.96875 72.81875) (end 115.77 72.81875) (width 0.2) (layer "F.Cu") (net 5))
 (segment (start 115.77 72.81875) (end 106.08625 82.5025) (width 0.2) (layer "F.Cu") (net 5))
 (segment (start 134.3025 79.80375) (end 134.3025 76.1525) (width 0.2) (layer "F.Cu") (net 5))
 (segment (start 134.3025 76.1525) (end 130.96875 72.81875) (width 0.2) (layer "F.Cu") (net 5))
 (segment (start 101.23325 73.8205) (end 90.01125 85.0425) (width 0.2) (layer "B.Cu") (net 3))
 (segment (start 147.36925 73.8205) (end 101.23325 73.8205) (width 0.2) (layer "B.Cu") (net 3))
 (segment (start 153.3525 79.80375) (end 147.36925 73.8205) (width 0.2) (layer "B.Cu") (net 3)))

